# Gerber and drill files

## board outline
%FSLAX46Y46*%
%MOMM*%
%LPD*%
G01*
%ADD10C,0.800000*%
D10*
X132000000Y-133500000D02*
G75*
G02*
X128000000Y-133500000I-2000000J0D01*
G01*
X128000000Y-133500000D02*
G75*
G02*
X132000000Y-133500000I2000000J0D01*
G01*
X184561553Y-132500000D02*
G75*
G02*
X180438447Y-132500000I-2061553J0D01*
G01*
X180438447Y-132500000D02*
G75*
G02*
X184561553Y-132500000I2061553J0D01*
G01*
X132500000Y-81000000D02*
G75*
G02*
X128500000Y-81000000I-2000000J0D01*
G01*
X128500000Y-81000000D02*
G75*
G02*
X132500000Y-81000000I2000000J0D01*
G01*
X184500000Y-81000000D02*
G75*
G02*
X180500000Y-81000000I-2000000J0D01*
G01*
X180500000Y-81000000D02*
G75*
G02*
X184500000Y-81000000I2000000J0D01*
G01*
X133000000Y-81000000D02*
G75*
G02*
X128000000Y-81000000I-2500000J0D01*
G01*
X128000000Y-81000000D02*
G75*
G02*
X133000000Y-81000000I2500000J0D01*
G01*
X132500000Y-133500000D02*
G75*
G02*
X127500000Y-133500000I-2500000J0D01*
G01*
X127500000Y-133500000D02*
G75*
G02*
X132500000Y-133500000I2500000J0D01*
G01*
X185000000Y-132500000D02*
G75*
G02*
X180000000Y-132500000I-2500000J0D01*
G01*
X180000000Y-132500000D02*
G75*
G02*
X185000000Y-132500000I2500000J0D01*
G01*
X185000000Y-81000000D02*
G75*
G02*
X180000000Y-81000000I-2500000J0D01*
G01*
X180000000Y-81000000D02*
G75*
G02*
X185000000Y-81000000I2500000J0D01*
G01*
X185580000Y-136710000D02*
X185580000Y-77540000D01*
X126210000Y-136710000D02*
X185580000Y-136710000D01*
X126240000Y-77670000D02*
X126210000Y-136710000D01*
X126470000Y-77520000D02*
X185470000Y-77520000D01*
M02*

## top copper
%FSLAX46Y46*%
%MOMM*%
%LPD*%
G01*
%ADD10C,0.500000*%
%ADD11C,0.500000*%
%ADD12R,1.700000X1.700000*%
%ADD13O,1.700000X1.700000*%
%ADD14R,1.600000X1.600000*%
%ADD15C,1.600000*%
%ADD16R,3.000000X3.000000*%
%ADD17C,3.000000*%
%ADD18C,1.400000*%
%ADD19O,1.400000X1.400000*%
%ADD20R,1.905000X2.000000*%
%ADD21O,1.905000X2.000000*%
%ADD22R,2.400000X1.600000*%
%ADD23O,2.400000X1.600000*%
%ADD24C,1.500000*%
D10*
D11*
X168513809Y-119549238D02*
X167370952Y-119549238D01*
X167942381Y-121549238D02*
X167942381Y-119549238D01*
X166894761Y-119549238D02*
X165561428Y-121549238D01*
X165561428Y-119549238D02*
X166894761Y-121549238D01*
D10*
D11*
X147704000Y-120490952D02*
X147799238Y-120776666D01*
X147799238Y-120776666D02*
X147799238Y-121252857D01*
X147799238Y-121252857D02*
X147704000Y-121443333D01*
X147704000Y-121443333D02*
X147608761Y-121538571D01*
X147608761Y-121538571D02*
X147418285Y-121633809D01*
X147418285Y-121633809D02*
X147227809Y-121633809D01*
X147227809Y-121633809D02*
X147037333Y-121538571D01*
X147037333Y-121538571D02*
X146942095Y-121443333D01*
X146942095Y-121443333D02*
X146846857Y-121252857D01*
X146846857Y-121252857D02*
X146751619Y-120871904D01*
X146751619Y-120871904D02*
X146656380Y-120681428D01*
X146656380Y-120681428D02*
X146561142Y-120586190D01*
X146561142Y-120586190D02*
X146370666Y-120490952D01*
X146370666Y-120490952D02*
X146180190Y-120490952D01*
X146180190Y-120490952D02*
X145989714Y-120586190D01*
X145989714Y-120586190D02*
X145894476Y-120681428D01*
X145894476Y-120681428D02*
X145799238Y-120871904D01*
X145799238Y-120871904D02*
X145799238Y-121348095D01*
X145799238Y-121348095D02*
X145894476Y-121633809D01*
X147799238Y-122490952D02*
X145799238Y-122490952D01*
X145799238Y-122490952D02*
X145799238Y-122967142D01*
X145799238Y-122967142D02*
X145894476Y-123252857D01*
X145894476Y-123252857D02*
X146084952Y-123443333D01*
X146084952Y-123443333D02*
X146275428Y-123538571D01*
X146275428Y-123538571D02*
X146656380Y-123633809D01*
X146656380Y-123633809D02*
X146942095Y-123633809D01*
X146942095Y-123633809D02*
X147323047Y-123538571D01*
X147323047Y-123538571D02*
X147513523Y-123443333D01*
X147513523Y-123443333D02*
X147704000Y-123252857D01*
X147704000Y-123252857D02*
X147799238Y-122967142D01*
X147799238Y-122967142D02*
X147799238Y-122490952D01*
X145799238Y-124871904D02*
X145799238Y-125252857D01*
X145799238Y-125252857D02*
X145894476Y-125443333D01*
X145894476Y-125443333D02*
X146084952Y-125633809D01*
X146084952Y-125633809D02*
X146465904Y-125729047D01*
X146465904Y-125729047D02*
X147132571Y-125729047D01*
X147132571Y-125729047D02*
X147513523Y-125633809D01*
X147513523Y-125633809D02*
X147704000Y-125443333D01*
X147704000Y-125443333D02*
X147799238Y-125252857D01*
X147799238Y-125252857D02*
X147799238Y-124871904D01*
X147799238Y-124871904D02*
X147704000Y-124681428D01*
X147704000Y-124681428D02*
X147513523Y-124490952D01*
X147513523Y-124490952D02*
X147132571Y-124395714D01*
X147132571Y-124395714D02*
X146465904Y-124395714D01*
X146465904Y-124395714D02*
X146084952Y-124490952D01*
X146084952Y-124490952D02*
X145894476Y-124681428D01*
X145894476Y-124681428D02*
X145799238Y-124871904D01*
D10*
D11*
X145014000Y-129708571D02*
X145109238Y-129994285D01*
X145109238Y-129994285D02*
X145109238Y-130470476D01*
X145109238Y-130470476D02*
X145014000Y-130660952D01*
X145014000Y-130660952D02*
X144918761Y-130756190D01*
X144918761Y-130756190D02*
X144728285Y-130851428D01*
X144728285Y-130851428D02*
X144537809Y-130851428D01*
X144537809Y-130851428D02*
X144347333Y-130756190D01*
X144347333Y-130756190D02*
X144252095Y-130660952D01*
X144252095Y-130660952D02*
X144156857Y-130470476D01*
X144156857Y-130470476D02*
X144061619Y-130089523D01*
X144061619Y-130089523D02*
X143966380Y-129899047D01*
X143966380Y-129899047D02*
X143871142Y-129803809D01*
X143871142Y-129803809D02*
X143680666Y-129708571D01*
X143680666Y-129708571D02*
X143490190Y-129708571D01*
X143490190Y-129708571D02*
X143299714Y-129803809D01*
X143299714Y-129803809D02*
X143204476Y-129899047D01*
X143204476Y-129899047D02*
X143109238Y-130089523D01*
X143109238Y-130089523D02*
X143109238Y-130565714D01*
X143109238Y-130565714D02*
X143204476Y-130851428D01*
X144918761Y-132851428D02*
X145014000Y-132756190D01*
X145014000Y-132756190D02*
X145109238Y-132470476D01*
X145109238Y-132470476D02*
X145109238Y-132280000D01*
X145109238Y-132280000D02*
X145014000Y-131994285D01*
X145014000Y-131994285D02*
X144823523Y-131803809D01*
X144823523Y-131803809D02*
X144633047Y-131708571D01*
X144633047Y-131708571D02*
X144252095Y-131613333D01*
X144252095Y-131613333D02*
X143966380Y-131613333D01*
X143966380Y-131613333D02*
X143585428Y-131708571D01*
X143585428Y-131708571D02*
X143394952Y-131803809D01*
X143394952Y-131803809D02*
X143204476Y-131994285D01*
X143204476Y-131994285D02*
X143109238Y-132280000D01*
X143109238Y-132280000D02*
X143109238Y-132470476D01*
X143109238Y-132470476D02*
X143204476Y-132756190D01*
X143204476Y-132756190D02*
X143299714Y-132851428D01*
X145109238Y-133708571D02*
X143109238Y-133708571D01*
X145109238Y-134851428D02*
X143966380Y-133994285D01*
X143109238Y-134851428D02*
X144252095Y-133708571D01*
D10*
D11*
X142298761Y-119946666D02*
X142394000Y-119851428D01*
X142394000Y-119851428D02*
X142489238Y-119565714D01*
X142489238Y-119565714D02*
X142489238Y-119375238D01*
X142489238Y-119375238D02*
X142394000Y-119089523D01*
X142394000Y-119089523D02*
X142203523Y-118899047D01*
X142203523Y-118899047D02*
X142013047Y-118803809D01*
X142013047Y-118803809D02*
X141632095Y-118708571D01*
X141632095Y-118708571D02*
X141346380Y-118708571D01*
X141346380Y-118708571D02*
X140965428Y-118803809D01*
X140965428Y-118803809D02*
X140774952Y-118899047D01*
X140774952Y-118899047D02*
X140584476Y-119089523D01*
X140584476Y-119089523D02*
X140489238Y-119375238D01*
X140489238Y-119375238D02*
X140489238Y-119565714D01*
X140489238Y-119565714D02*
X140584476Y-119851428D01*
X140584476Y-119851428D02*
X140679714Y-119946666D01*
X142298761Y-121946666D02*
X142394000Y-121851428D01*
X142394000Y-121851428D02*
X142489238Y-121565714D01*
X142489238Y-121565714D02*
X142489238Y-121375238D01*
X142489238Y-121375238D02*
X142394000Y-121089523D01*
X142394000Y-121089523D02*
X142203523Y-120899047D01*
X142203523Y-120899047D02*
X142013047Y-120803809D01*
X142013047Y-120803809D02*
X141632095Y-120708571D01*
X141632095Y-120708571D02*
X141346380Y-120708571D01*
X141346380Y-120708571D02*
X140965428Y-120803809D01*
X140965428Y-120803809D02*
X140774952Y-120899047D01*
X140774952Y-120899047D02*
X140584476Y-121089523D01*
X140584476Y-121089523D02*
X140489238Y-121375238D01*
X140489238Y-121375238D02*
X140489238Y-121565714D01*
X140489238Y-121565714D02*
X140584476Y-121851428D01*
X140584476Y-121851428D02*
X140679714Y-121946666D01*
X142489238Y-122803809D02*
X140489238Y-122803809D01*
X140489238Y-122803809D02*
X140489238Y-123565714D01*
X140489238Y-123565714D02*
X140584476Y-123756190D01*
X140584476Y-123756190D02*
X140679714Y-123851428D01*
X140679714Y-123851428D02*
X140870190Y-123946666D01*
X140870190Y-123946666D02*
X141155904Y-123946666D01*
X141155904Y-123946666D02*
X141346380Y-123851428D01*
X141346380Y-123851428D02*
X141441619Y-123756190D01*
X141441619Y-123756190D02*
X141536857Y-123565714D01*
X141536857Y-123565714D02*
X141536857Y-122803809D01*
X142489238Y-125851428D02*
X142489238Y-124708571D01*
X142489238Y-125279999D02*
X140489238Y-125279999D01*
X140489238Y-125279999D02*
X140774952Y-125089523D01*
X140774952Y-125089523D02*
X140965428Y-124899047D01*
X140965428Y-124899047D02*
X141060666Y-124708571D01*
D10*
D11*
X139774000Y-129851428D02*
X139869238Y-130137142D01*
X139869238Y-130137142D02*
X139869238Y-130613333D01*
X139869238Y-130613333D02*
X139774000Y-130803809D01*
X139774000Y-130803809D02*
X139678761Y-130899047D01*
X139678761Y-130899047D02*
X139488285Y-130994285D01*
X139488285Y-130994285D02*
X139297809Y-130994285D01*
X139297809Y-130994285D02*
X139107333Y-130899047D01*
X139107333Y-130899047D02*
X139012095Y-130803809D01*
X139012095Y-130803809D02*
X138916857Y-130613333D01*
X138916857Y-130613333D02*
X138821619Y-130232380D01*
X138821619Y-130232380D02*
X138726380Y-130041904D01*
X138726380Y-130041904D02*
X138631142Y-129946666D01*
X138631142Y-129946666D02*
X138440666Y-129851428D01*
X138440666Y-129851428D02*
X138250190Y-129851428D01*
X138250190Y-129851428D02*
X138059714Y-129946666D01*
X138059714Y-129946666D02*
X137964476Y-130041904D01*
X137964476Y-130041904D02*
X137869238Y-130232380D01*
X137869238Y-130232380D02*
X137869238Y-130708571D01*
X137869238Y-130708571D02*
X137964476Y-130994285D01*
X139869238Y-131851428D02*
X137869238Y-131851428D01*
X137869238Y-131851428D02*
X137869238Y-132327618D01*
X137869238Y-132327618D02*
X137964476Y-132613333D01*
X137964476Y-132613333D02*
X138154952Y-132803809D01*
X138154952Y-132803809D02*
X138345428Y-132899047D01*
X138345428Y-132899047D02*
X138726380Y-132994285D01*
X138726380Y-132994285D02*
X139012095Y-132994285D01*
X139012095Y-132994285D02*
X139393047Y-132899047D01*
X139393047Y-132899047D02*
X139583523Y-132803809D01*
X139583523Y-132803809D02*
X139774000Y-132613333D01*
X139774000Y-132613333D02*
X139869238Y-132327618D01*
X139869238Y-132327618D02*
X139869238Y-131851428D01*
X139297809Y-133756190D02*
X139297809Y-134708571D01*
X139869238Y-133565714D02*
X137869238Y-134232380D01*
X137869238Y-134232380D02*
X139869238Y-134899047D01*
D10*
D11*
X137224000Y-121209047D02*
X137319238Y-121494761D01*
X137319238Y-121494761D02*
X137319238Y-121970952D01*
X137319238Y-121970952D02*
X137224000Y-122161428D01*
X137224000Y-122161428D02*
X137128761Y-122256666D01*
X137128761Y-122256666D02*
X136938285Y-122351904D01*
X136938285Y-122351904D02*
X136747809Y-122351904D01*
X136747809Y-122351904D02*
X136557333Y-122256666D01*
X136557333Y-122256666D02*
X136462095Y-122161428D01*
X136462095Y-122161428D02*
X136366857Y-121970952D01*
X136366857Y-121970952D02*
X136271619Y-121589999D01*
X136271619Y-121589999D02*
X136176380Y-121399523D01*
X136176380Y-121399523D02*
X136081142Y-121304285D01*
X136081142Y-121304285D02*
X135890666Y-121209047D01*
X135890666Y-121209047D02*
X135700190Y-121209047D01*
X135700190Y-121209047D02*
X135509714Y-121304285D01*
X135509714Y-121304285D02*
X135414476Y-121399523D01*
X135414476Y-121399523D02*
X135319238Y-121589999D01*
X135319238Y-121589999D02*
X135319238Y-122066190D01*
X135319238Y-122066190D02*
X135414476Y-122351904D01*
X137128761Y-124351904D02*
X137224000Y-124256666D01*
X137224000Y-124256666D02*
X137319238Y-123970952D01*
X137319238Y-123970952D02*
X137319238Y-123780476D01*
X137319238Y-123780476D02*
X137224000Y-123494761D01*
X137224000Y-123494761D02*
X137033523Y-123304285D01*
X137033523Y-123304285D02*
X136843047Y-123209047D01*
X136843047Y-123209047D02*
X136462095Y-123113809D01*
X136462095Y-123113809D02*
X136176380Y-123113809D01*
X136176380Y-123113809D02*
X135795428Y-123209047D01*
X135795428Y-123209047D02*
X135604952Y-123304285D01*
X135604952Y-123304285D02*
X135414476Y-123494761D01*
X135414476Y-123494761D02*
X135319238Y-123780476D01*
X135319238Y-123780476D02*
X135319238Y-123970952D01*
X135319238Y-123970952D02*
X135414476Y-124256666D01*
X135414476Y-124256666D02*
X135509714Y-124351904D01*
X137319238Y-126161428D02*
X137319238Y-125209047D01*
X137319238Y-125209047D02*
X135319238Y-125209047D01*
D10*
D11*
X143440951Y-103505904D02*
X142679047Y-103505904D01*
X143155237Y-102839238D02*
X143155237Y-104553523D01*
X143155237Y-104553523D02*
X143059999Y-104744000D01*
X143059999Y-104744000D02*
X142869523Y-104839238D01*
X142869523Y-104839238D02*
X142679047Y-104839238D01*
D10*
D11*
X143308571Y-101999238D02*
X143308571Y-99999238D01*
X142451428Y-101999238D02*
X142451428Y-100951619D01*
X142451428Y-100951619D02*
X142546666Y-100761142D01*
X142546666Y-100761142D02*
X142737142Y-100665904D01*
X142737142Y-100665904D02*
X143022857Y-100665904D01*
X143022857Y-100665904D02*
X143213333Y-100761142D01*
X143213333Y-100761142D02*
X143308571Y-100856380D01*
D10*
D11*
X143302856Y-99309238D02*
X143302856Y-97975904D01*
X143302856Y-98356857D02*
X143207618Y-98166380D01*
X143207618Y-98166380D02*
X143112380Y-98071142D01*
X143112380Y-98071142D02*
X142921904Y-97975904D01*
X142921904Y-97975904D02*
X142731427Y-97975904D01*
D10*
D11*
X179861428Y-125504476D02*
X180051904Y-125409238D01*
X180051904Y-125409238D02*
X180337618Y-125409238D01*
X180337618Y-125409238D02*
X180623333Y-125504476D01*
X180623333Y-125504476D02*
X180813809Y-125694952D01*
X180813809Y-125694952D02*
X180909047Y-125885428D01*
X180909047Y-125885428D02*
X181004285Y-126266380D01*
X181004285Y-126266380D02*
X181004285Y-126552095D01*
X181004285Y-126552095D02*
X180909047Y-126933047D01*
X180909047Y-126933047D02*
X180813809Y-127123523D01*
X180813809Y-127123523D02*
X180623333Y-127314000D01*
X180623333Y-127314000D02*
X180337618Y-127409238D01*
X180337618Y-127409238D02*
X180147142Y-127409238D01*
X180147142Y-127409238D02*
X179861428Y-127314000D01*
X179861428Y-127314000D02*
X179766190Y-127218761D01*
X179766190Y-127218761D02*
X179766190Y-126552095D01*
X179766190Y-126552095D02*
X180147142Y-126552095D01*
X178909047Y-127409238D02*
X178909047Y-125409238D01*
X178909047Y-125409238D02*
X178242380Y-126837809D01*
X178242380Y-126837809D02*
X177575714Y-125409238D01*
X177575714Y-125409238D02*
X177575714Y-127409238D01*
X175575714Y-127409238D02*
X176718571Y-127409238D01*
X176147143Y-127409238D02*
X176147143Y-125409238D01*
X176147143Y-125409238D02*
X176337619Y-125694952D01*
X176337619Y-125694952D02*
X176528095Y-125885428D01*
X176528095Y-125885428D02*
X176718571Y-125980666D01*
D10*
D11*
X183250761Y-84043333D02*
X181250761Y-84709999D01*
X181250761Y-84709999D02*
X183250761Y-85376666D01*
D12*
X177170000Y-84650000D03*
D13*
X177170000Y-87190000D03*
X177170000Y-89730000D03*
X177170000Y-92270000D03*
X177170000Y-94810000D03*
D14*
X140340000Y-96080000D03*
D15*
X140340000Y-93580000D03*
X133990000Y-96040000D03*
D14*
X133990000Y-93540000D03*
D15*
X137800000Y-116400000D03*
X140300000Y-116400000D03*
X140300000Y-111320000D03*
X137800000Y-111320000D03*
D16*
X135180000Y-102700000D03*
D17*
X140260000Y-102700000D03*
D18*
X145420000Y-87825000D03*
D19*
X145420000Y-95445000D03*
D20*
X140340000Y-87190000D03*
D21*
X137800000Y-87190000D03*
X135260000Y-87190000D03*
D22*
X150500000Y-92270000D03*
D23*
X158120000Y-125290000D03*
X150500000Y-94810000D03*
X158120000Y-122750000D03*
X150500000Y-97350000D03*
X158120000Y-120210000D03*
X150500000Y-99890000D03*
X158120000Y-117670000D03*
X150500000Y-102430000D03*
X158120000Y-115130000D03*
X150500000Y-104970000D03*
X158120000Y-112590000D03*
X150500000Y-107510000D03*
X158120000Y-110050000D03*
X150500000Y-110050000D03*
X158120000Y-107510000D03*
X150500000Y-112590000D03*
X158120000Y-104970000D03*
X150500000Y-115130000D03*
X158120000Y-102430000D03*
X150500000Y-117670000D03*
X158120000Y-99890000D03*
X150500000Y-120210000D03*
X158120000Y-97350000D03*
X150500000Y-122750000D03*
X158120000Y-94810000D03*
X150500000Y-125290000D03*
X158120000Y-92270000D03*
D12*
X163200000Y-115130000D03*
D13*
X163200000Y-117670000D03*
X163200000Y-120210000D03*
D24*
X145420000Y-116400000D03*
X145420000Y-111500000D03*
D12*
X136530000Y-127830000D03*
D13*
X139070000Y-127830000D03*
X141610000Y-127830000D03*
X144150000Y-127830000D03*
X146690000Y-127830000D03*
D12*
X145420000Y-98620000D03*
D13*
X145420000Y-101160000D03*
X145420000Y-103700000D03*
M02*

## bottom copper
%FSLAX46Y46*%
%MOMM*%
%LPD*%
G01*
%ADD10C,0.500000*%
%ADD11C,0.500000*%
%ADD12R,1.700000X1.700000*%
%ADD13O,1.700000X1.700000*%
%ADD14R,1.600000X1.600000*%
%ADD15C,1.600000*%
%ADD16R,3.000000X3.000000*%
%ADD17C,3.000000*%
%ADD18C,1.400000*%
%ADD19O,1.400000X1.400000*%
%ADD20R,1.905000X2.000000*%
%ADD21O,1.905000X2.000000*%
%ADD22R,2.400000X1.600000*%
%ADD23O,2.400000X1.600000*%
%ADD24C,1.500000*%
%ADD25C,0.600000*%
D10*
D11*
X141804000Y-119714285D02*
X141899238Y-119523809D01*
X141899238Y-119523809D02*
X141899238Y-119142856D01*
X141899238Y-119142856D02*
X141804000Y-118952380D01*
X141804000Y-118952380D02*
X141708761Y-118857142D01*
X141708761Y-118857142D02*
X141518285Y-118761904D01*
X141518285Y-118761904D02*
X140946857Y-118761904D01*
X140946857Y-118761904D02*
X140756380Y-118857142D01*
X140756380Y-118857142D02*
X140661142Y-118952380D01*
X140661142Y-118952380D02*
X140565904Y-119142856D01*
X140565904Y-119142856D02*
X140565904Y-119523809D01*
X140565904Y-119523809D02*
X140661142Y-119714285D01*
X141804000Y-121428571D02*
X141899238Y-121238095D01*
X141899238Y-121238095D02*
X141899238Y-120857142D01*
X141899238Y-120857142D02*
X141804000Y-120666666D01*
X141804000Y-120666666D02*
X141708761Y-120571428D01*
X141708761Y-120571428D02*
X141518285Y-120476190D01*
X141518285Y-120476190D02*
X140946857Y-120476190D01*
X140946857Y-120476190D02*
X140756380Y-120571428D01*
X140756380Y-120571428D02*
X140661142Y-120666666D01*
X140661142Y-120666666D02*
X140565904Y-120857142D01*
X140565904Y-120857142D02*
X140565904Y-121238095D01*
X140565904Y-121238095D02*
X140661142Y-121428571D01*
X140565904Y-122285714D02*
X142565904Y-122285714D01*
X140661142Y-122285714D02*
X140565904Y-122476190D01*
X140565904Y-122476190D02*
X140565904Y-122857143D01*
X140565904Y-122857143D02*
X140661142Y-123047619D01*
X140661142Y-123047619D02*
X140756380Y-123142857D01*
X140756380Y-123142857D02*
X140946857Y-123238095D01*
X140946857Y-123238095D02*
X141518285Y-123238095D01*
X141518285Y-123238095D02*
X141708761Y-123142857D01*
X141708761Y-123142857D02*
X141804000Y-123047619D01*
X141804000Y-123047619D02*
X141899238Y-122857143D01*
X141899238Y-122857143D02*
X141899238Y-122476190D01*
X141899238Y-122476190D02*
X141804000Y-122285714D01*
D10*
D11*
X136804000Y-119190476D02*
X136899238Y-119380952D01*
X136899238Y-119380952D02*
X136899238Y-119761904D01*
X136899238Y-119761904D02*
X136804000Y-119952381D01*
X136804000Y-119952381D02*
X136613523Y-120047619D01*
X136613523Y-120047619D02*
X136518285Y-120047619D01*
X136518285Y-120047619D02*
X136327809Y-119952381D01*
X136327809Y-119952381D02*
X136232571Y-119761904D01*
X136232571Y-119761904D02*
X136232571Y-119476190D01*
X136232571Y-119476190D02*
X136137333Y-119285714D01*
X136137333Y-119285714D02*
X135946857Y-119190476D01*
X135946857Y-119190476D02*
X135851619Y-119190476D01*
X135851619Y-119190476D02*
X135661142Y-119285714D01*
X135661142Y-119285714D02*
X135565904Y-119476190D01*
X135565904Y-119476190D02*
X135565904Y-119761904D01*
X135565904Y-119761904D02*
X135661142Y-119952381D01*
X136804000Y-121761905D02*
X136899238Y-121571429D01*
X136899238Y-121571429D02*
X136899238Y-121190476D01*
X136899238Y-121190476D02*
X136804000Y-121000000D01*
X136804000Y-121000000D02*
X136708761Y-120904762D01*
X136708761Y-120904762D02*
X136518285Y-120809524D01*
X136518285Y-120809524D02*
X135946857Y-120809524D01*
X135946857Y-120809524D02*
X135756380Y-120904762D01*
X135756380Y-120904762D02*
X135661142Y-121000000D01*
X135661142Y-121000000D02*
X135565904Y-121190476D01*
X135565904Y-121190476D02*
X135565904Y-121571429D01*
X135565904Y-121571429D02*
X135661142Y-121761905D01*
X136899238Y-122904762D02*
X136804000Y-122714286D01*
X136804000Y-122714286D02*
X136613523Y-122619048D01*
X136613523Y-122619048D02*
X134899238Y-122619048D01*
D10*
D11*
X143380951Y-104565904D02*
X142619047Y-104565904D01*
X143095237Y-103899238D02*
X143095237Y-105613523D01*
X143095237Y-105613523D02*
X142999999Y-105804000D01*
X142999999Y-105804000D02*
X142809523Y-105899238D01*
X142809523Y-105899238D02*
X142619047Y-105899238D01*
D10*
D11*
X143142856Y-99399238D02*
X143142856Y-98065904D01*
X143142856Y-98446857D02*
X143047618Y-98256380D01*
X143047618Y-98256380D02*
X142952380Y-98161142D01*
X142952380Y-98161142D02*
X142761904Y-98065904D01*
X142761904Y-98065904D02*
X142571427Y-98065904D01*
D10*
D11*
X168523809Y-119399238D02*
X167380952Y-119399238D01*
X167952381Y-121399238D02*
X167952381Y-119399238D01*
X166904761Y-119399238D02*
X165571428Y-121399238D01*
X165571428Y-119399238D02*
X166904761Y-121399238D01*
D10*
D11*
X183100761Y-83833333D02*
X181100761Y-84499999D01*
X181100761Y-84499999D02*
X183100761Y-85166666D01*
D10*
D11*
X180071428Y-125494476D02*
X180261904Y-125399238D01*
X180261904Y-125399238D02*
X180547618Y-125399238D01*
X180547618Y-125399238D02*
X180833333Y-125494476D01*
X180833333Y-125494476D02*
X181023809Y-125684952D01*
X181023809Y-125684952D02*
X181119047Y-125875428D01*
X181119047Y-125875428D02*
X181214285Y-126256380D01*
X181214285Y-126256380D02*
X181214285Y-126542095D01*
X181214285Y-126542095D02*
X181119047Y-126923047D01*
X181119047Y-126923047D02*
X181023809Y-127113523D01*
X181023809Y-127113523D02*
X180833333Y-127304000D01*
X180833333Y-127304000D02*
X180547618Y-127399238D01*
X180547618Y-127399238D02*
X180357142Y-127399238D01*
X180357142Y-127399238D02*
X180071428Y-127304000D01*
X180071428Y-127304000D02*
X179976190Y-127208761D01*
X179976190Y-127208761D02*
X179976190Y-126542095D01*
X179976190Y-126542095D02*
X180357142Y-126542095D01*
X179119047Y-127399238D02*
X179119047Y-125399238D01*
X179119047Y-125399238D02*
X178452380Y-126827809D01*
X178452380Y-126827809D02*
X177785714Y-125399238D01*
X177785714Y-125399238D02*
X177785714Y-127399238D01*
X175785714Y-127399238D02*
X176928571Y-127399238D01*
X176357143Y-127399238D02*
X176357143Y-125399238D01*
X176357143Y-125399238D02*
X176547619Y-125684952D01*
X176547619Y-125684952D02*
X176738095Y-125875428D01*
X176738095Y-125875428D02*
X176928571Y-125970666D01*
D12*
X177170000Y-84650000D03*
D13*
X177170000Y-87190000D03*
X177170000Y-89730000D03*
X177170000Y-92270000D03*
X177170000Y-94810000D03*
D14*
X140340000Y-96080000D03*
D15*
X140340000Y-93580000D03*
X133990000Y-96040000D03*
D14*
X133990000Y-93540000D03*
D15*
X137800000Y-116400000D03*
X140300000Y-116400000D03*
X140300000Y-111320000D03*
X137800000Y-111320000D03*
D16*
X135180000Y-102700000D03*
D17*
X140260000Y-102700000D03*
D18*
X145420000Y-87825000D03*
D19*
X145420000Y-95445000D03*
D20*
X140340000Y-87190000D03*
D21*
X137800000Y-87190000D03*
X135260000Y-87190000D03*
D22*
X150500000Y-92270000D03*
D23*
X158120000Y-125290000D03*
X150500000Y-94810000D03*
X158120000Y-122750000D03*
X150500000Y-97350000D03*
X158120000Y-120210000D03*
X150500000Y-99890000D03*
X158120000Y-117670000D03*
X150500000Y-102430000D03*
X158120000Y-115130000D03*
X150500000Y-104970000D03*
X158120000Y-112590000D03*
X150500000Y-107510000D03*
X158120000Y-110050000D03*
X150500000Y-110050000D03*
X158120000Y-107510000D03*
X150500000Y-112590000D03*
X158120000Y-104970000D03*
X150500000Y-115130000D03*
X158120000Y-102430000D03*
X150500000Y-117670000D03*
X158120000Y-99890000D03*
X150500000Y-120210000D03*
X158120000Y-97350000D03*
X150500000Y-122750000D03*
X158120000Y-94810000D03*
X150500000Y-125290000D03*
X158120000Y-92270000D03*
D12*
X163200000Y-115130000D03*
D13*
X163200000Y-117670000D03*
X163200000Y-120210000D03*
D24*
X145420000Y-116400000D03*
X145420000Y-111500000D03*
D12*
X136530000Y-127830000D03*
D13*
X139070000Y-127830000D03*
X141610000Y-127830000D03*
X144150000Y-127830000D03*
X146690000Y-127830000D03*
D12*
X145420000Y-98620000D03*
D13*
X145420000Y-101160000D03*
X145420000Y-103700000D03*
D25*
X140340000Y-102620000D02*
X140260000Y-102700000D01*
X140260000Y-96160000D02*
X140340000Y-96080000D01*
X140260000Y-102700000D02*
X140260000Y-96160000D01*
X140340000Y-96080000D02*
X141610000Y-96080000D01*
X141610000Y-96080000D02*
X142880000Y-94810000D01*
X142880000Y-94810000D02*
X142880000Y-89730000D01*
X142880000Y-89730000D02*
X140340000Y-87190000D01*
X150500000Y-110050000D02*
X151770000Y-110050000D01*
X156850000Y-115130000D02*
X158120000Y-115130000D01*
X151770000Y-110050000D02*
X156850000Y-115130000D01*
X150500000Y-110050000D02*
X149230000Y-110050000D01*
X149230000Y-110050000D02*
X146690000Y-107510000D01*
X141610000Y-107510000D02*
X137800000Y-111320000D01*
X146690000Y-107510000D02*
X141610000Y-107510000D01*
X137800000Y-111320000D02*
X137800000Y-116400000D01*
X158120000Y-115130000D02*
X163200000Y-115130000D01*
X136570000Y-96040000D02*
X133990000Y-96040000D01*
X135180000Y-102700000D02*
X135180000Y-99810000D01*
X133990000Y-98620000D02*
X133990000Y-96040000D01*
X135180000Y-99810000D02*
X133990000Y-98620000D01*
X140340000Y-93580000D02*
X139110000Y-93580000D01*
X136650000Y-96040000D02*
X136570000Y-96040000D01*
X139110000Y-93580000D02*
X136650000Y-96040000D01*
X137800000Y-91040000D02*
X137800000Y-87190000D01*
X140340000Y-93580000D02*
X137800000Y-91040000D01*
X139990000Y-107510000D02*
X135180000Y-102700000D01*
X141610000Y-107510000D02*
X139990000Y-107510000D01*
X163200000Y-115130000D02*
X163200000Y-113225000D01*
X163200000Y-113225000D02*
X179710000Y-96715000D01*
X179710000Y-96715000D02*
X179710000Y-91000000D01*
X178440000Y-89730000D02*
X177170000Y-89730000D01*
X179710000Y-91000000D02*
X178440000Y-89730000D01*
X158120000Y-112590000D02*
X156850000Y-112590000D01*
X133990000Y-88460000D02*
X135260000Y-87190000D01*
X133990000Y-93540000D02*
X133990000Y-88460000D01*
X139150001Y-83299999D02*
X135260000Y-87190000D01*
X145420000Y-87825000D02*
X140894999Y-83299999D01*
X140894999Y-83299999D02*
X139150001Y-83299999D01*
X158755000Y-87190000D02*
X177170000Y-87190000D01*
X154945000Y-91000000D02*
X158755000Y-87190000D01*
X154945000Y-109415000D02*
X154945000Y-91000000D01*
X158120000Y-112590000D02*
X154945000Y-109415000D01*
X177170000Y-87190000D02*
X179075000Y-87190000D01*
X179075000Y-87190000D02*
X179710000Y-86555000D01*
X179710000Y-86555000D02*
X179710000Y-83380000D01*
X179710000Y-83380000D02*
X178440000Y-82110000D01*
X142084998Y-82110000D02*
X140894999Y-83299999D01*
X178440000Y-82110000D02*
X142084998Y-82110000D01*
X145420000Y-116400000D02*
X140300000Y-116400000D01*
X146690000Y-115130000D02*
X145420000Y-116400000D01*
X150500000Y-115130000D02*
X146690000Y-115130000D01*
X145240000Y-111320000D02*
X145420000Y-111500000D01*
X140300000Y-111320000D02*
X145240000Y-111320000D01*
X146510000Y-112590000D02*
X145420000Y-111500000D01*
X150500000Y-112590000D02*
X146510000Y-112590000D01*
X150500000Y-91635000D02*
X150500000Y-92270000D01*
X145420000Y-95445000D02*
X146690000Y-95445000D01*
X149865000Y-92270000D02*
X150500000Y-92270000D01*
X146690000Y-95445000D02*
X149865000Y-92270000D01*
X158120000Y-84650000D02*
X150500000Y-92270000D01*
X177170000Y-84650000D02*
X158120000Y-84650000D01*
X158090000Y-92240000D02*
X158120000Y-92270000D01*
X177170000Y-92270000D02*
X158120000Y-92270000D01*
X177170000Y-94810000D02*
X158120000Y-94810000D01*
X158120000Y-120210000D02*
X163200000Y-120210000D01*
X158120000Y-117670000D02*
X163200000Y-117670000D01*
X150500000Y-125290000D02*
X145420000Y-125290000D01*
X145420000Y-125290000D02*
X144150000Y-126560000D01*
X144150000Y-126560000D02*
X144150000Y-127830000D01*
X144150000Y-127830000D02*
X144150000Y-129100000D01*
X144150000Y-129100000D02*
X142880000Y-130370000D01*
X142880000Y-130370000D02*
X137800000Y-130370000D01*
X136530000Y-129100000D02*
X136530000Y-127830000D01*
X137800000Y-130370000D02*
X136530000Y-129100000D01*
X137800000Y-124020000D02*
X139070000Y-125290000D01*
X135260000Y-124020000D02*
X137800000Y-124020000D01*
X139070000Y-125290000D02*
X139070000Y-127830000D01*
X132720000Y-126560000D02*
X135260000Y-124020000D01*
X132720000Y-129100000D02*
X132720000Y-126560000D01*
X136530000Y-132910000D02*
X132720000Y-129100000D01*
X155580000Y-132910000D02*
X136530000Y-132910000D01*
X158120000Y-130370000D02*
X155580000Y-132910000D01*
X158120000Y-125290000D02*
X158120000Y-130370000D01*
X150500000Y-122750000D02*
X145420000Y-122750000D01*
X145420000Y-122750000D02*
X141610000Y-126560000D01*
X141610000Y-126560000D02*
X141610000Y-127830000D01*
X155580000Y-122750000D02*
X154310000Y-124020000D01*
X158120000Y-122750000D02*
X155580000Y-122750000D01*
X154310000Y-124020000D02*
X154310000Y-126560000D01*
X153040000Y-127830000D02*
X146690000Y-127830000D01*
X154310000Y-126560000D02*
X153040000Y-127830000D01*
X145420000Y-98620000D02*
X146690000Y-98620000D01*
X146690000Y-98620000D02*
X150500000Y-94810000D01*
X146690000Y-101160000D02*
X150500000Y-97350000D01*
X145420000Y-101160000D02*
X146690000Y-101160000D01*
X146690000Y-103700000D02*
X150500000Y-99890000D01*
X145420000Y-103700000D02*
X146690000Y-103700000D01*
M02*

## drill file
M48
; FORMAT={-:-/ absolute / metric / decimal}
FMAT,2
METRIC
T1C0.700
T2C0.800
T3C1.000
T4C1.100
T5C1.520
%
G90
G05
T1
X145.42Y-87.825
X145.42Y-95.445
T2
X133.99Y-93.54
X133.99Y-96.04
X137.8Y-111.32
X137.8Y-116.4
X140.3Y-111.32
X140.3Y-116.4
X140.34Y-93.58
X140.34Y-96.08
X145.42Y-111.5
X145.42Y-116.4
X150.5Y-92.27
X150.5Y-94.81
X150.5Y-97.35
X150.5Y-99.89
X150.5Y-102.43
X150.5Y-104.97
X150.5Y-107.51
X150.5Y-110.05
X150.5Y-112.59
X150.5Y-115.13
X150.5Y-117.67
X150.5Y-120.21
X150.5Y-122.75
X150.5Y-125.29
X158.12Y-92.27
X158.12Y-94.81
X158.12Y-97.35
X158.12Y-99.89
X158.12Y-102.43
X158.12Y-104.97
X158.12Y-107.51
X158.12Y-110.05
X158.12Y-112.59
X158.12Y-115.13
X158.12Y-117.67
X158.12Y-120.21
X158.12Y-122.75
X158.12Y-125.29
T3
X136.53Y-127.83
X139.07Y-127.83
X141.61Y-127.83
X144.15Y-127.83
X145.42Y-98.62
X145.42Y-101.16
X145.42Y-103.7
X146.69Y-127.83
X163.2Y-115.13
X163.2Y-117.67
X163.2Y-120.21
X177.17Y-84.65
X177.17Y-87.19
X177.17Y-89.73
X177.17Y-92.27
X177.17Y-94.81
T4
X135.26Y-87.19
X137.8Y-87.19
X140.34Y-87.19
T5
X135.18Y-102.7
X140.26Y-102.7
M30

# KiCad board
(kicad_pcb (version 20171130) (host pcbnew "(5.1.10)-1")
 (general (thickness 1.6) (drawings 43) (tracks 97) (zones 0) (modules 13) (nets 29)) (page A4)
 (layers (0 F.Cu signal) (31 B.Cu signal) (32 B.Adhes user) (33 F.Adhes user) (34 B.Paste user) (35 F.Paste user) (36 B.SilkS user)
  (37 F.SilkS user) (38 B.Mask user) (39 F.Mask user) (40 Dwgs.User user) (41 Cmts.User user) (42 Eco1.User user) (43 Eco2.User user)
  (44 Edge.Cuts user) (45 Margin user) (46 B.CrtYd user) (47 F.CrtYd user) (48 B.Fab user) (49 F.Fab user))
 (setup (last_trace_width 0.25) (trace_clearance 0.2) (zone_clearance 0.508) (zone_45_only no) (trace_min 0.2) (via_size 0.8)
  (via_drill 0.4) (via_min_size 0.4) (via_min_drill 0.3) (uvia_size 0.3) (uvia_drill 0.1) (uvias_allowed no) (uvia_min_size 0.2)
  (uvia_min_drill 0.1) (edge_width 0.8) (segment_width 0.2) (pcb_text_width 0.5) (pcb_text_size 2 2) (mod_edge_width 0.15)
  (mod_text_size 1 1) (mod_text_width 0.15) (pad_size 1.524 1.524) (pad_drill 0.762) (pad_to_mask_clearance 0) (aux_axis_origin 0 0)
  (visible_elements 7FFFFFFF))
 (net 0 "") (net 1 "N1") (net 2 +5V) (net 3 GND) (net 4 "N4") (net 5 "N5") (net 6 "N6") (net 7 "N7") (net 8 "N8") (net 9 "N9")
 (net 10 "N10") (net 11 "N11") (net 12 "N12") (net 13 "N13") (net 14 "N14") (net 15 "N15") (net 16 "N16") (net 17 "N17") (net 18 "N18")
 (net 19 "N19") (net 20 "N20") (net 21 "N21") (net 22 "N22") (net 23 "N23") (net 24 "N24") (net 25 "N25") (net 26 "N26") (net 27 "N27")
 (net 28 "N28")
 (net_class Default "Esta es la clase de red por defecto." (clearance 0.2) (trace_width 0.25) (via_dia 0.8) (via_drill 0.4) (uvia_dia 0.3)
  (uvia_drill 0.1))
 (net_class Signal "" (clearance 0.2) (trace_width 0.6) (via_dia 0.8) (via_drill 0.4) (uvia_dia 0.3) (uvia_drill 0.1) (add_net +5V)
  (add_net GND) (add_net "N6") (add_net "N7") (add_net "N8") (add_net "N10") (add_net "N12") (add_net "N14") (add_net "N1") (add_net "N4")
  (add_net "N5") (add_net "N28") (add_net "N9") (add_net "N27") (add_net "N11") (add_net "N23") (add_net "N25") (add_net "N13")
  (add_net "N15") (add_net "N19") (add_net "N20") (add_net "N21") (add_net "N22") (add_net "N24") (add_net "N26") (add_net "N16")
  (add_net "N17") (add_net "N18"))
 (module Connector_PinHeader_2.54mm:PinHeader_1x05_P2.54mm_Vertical (layer F.Cu) (at 177.17 84.65)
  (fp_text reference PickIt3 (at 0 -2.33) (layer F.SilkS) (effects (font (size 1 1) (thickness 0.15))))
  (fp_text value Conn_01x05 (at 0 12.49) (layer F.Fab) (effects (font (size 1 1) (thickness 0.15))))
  (pad 1 thru_hole rect (at 0 0) (size 1.7 1.7) (drill 1) (layers *.Cu *.Mask) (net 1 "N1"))
  (pad 2 thru_hole oval (at 0 2.54) (size 1.7 1.7) (drill 1) (layers *.Cu *.Mask) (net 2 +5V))
  (pad 3 thru_hole oval (at 0 5.08) (size 1.7 1.7) (drill 1) (layers *.Cu *.Mask) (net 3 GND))
  (pad 4 thru_hole oval (at 0 7.62) (size 1.7 1.7) (drill 1) (layers *.Cu *.Mask) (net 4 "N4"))
  (pad 5 thru_hole oval (at 0 10.16) (size 1.7 1.7) (drill 1) (layers *.Cu *.Mask) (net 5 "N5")))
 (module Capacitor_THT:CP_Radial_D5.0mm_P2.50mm (layer F.Cu) (at 140.34 96.08 90)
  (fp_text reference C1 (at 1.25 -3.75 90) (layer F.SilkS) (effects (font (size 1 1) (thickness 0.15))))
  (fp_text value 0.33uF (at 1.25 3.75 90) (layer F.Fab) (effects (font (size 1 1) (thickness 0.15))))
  (pad 1 thru_hole rect (at 0 0 90) (size 1.6 1.6) (drill 0.8) (layers *.Cu *.Mask) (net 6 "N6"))
  (pad 2 thru_hole circle (at 2.5 0 90) (size 1.6 1.6) (drill 0.8) (layers *.Cu *.Mask) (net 3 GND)))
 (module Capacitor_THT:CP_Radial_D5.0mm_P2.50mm (layer F.Cu) (at 133.99 93.54 270)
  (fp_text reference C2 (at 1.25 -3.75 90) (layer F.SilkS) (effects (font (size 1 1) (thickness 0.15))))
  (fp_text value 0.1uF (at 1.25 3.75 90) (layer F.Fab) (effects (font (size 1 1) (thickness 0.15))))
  (pad 2 thru_hole circle (at 2.5 0 270) (size 1.6 1.6) (drill 0.8) (layers *.Cu *.Mask) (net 3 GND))
  (pad 1 thru_hole rect (at 0 0 270) (size 1.6 1.6) (drill 0.8) (layers *.Cu *.Mask) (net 2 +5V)))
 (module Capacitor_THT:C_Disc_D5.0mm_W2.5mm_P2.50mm (layer F.Cu) (at 137.8 116.4)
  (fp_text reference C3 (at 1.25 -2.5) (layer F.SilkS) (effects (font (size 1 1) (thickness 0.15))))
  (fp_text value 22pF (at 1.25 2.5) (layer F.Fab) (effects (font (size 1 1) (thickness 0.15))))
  (pad 1 thru_hole circle (at 0 0) (size 1.6 1.6) (drill 0.8) (layers *.Cu *.Mask) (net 3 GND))
  (pad 2 thru_hole circle (at 2.5 0) (size 1.6 1.6) (drill 0.8) (layers *.Cu *.Mask) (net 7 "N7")))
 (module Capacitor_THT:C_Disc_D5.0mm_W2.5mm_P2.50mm (layer F.Cu) (at 137.8 111.32)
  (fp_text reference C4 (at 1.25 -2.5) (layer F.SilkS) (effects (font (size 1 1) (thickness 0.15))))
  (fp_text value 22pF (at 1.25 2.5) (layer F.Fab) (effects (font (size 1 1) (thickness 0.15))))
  (pad 2 thru_hole circle (at 2.5 0) (size 1.6 1.6) (drill 0.8) (layers *.Cu *.Mask) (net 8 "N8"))
  (pad 1 thru_hole circle (at 0 0) (size 1.6 1.6) (drill 0.8) (layers *.Cu *.Mask) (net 3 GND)))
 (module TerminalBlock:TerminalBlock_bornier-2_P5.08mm (layer F.Cu) (at 135.18 102.7)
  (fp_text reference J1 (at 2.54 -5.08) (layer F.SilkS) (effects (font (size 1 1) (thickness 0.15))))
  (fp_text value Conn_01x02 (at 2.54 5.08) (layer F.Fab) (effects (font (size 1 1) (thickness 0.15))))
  (pad 1 thru_hole rect (at 0 0) (size 3 3) (drill 1.52) (layers *.Cu *.Mask) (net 3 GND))
  (pad 2 thru_hole circle (at 5.08 0) (size 3 3) (drill 1.52) (layers *.Cu *.Mask) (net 6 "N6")))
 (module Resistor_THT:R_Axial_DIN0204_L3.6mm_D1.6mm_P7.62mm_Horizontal (layer F.Cu) (at 145.42 87.825 270)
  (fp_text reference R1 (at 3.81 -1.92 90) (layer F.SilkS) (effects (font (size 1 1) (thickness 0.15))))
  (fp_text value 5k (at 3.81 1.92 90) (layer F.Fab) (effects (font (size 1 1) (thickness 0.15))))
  (pad 1 thru_hole circle (at 0 0 270) (size 1.4 1.4) (drill 0.7) (layers *.Cu *.Mask) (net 2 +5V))
  (pad 2 thru_hole oval (at 7.62 0 270) (size 1.4 1.4) (drill 0.7) (layers *.Cu *.Mask) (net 1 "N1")))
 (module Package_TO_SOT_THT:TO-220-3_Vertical (layer F.Cu) (at 140.34 87.19 180)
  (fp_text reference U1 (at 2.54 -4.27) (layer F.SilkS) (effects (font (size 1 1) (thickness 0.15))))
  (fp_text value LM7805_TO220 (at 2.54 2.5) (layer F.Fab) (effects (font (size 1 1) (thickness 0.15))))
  (pad 1 thru_hole rect (at 0 0 180) (size 1.905 2) (drill 1.1) (layers *.Cu *.Mask) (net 6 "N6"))
  (pad 2 thru_hole oval (at 2.54 0 180) (size 1.905 2) (drill 1.1) (layers *.Cu *.Mask) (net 3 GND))
  (pad 3 thru_hole oval (at 5.08 0 180) (size 1.905 2) (drill 1.1) (layers *.Cu *.Mask) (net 2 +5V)))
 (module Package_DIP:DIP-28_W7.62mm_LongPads (layer F.Cu) (at 150.5 92.27)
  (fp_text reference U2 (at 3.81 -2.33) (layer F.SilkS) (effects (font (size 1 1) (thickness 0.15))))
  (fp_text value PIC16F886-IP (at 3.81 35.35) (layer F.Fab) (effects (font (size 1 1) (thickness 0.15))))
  (pad 1 thru_hole rect (at 0 0) (size 2.4 1.6) (drill 0.8) (layers *.Cu *.Mask) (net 1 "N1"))
  (pad 15 thru_hole oval (at 7.62 33.02) (size 2.4 1.6) (drill 0.8) (layers *.Cu *.Mask) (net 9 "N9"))
  (pad 2 thru_hole oval (at 0 2.54) (size 2.4 1.6) (drill 0.8) (layers *.Cu *.Mask) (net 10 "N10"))
  (pad 16 thru_hole oval (at 7.62 30.48) (size 2.4 1.6) (drill 0.8) (layers *.Cu *.Mask) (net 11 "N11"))
  (pad 3 thru_hole oval (at 0 5.08) (size 2.4 1.6) (drill 0.8) (layers *.Cu *.Mask) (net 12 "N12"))
  (pad 17 thru_hole oval (at 7.62 27.94) (size 2.4 1.6) (drill 0.8) (layers *.Cu *.Mask) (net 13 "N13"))
  (pad 4 thru_hole oval (at 0 7.62) (size 2.4 1.6) (drill 0.8) (layers *.Cu *.Mask) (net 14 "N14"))
  (pad 18 thru_hole oval (at 7.62 25.4) (size 2.4 1.6) (drill 0.8) (layers *.Cu *.Mask) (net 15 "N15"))
  (pad 5 thru_hole oval (at 0 10.16) (size 2.4 1.6) (drill 0.8) (layers *.Cu *.Mask) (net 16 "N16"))
  (pad 19 thru_hole oval (at 7.62 22.86) (size 2.4 1.6) (drill 0.8) (layers *.Cu *.Mask) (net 3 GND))
  (pad 6 thru_hole oval (at 0 12.7) (size 2.4 1.6) (drill 0.8) (layers *.Cu *.Mask) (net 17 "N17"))
  (pad 20 thru_hole oval (at 7.62 20.32) (size 2.4 1.6) (drill 0.8) (layers *.Cu *.Mask) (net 2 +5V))
  (pad 7 thru_hole oval (at 0 15.24) (size 2.4 1.6) (drill 0.8) (layers *.Cu *.Mask) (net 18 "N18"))
  (pad 21 thru_hole oval (at 7.62 17.78) (size 2.4 1.6) (drill 0.8) (layers *.Cu *.Mask) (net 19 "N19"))
  (pad 8 thru_hole oval (at 0 17.78) (size 2.4 1.6) (drill 0.8) (layers *.Cu *.Mask) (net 3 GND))
  (pad 22 thru_hole oval (at 7.62 15.24) (size 2.4 1.6) (drill 0.8) (layers *.Cu *.Mask) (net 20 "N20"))
  (pad 9 thru_hole oval (at 0 20.32) (size 2.4 1.6) (drill 0.8) (layers *.Cu *.Mask) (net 8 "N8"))
  (pad 23 thru_hole oval (at 7.62 12.7) (size 2.4 1.6) (drill 0.8) (layers *.Cu *.Mask) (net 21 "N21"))
  (pad 10 thru_hole oval (at 0 22.86) (size 2.4 1.6) (drill 0.8) (layers *.Cu *.Mask) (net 7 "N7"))
  (pad 24 thru_hole oval (at 7.62 10.16) (size 2.4 1.6) (drill 0.8) (layers *.Cu *.Mask) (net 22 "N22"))
  (pad 11 thru_hole oval (at 0 25.4) (size 2.4 1.6) (drill 0.8) (layers *.Cu *.Mask) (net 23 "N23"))
  (pad 25 thru_hole oval (at 7.62 7.62) (size 2.4 1.6) (drill 0.8) (layers *.Cu *.Mask) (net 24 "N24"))
  (pad 12 thru_hole oval (at 0 27.94) (size 2.4 1.6) (drill 0.8) (layers *.Cu *.Mask) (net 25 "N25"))
  (pad 26 thru_hole oval (at 7.62 5.08) (size 2.4 1.6) (drill 0.8) (layers *.Cu *.Mask) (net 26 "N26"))
  (pad 13 thru_hole oval (at 0 30.48) (size 2.4 1.6) (drill 0.8) (layers *.Cu *.Mask) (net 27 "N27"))
  (pad 27 thru_hole oval (at 7.62 2.54) (size 2.4 1.6) (drill 0.8) (layers *.Cu *.Mask) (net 5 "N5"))
  (pad 14 thru_hole oval (at 0 33.02) (size 2.4 1.6) (drill 0.8) (layers *.Cu *.Mask) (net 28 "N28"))
  (pad 28 thru_hole oval (at 7.62 0) (size 2.4 1.6) (drill 0.8) (layers *.Cu *.Mask) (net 4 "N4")))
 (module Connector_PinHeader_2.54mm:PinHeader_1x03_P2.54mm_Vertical (layer F.Cu) (at 163.2 115.13)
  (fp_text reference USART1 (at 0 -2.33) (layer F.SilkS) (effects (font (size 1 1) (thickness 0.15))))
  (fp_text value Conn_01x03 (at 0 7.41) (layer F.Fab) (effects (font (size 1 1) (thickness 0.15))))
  (pad 1 thru_hole rect (at 0 0) (size 1.7 1.7) (drill 1) (layers *.Cu *.Mask) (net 3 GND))
  (pad 2 thru_hole oval (at 0 2.54) (size 1.7 1.7) (drill 1) (layers *.Cu *.Mask) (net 15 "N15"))
  (pad 3 thru_hole oval (at 0 5.08) (size 1.7 1.7) (drill 1) (layers *.Cu *.Mask) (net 13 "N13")))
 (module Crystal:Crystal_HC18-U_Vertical (layer F.Cu) (at 145.42 116.4 90)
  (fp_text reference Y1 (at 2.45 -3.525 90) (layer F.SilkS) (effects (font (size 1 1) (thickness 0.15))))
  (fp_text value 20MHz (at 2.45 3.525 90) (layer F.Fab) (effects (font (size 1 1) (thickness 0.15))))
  (pad 1 thru_hole circle (at 0 0 90) (size 1.5 1.5) (drill 0.8) (layers *.Cu *.Mask) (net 7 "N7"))
  (pad 2 thru_hole circle (at 4.9 0 90) (size 1.5 1.5) (drill 0.8) (layers *.Cu *.Mask) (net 8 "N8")))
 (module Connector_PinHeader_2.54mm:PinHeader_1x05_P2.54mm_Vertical (layer F.Cu) (at 136.53 127.83 90)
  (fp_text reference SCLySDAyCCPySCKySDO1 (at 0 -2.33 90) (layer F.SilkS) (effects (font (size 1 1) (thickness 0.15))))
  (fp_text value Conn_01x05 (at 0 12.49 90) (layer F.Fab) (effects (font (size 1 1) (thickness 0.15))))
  (pad 1 thru_hole rect (at 0 0 90) (size 1.7 1.7) (drill 1) (layers *.Cu *.Mask) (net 28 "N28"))
  (pad 2 thru_hole oval (at 0 2.54 90) (size 1.7 1.7) (drill 1) (layers *.Cu *.Mask) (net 9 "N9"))
  (pad 3 thru_hole oval (at 0 5.08 90) (size 1.7 1.7) (drill 1) (layers *.Cu *.Mask) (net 27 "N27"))
  (pad 4 thru_hole oval (at 0 7.62 90) (size 1.7 1.7) (drill 1) (layers *.Cu *.Mask) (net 28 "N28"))
  (pad 5 thru_hole oval (at 0 10.16 90) (size 1.7 1.7) (drill 1) (layers *.Cu *.Mask) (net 11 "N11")))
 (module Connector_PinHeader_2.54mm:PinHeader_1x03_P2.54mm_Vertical (layer F.Cu) (at 145.42 98.62)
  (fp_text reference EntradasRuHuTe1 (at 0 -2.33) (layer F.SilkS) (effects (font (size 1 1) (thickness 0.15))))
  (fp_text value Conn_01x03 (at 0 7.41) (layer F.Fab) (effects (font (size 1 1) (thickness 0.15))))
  (pad 1 thru_hole rect (at 0 0) (size 1.7 1.7) (drill 1) (layers *.Cu *.Mask) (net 10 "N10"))
  (pad 2 thru_hole oval (at 0 2.54) (size 1.7 1.7) (drill 1) (layers *.Cu *.Mask) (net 12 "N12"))
  (pad 3 thru_hole oval (at 0 5.08) (size 1.7 1.7) (drill 1) (layers *.Cu *.Mask) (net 14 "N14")))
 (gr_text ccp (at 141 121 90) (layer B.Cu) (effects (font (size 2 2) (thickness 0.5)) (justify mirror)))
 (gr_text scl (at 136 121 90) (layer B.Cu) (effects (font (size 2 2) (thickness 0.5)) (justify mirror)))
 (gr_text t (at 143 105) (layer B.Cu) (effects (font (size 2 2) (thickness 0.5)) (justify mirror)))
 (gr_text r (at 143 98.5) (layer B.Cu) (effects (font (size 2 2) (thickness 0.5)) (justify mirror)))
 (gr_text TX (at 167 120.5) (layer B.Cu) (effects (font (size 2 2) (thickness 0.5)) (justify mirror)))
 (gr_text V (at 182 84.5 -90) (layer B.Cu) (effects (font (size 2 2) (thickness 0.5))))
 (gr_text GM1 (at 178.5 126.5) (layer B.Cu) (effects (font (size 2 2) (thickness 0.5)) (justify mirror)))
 (gr_circle (center 130 133.5) (end 132 133.5) (layer Edge.Cuts) (width 0.8))
 (gr_circle (center 182.5 132.5) (end 184.5 133) (layer Edge.Cuts) (width 0.8))
 (gr_circle (center 130.5 81) (end 132.5 81) (layer Edge.Cuts) (width 0.8))
 (gr_circle (center 182.5 81) (end 184.5 81) (layer Edge.Cuts) (width 0.8))
 (gr_circle (center 130.5 81) (end 133 81) (layer Edge.Cuts) (width 0.8))
 (gr_circle (center 130 133.5) (end 132.5 133.5) (layer Edge.Cuts) (width 0.8))
 (gr_circle (center 182.5 132.5) (end 185 132.5) (layer Edge.Cuts) (width 0.8))
 (gr_circle (center 182.5 81) (end 185 81) (layer Edge.Cuts) (width 0.8))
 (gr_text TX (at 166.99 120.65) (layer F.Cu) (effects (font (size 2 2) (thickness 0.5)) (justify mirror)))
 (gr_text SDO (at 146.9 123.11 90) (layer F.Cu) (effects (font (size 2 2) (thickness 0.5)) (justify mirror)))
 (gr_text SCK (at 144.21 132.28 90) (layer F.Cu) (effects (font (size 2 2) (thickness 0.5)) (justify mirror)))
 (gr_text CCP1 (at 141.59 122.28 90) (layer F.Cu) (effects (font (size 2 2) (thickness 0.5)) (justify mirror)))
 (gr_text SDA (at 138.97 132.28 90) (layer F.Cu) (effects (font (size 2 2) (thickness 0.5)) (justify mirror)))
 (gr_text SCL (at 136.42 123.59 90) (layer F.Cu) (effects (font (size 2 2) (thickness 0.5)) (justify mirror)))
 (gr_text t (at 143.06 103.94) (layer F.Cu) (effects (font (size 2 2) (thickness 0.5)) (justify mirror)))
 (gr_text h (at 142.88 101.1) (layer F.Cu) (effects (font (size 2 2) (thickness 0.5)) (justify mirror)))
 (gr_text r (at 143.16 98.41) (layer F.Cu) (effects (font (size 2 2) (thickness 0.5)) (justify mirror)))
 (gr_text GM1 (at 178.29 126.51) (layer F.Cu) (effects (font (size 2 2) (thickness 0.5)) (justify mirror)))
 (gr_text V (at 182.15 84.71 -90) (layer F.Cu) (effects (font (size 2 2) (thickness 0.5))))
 (gr_line (start 185.58 136.71) (end 185.58 77.54) (layer Edge.Cuts) (width 0.8))
 (gr_line (start 126.21 136.71) (end 185.58 136.71) (layer Edge.Cuts) (width 0.8))
 (gr_line (start 126.24 77.67) (end 126.21 136.71) (layer Edge.Cuts) (width 0.8))
 (gr_line (start 126.47 77.52) (end 185.47 77.52) (layer Edge.Cuts) (width 0.8))
 (segment (start 140.34 102.62) (end 140.26 102.7) (width 0.6) (layer B.Cu) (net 6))
 (segment (start 140.26 96.16) (end 140.34 96.08) (width 0.6) (layer B.Cu) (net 6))
 (segment (start 140.26 102.7) (end 140.26 96.16) (width 0.6) (layer B.Cu) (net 6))
 (segment (start 140.34 96.08) (end 141.61 96.08) (width 0.6) (layer B.Cu) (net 6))
 (segment (start 141.61 96.08) (end 142.88 94.81) (width 0.6) (layer B.Cu) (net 6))
 (segment (start 142.88 94.81) (end 142.88 89.73) (width 0.6) (layer B.Cu) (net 6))
 (segment (start 142.88 89.73) (end 140.34 87.19) (width 0.6) (layer B.Cu) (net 6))
 (segment (start 150.5 110.05) (end 151.77 110.05) (width 0.6) (layer B.Cu) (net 3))
 (segment (start 156.85 115.13) (end 158.12 115.13) (width 0.6) (layer B.Cu) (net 3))
 (segment (start 151.77 110.05) (end 156.85 115.13) (width 0.6) (layer B.Cu) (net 3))
 (segment (start 150.5 110.05) (end 149.23 110.05) (width 0.6) (layer B.Cu) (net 3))
 (segment (start 149.23 110.05) (end 146.69 107.51) (width 0.6) (layer B.Cu) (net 3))
 (segment (start 141.61 107.51) (end 137.8 111.32) (width 0.6) (layer B.Cu) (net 3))
 (segment (start 146.69 107.51) (end 141.61 107.51) (width 0.6) (layer B.Cu) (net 3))
 (segment (start 137.8 111.32) (end 137.8 116.4) (width 0.6) (layer B.Cu) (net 3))
 (segment (start 158.12 115.13) (end 163.2 115.13) (width 0.6) (layer B.Cu) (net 3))
 (segment (start 136.57 96.04) (end 133.99 96.04) (width 0.6) (layer B.Cu) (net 3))
 (segment (start 135.18 102.7) (end 135.18 99.81) (width 0.6) (layer B.Cu) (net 3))
 (segment (start 133.99 98.62) (end 133.99 96.04) (width 0.6) (layer B.Cu) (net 3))
 (segment (start 135.18 99.81) (end 133.99 98.62) (width 0.6) (layer B.Cu) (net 3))
 (segment (start 140.34 93.58) (end 139.11 93.58) (width 0.6) (layer B.Cu) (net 3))
 (segment (start 136.65 96.04) (end 136.57 96.04) (width 0.6) (layer B.Cu) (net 3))
 (segment (start 139.11 93.58) (end 136.65 96.04) (width 0.6) (layer B.Cu) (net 3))
 (segment (start 137.8 91.04) (end 137.8 87.19) (width 0.6) (layer B.Cu) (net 3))
 (segment (start 140.34 93.58) (end 137.8 91.04) (width 0.6) (layer B.Cu) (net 3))
 (segment (start 139.99 107.51) (end 135.18 102.7) (width 0.6) (layer B.Cu) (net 3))
 (segment (start 141.61 107.51) (end 139.99 107.51) (width 0.6) (layer B.Cu) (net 3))
 (segment (start 163.2 115.13) (end 163.2 113.225) (width 0.6) (layer B.Cu) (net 3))
 (segment (start 163.2 113.225) (end 179.71 96.715) (width 0.6) (layer B.Cu) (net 3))
 (segment (start 179.71 96.715) (end 179.71 91) (width 0.6) (layer B.Cu) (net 3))
 (segment (start 178.44 89.73) (end 177.17 89.73) (width 0.6) (layer B.Cu) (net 3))
 (segment (start 179.71 91) (end 178.44 89.73) (width 0.6) (layer B.Cu) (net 3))
 (segment (start 158.12 112.59) (end 156.85 112.59) (width 0.6) (layer B.Cu) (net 2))
 (segment (start 133.99 88.46) (end 135.26 87.19) (width 0.6) (layer B.Cu) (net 2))
 (segment (start 133.99 93.54) (end 133.99 88.46) (width 0.6) (layer B.Cu) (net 2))
 (segment (start 139.150001 83.299999) (end 135.26 87.19) (width 0.6) (layer B.Cu) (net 2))
 (segment (start 145.42 87.825) (end 140.894999 83.299999) (width 0.6) (layer B.Cu) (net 2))
 (segment (start 140.894999 83.299999) (end 139.150001 83.299999) (width 0.6) (layer B.Cu) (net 2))
 (segment (start 158.755 87.19) (end 177.17 87.19) (width 0.6) (layer B.Cu) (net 2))
 (segment (start 154.945 91) (end 158.755 87.19) (width 0.6) (layer B.Cu) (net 2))
 (segment (start 154.945 109.415) (end 154.945 91) (width 0.6) (layer B.Cu) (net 2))
 (segment (start 158.12 112.59) (end 154.945 109.415) (width 0.6) (layer B.Cu) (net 2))
 (segment (start 177.17 87.19) (end 179.075 87.19) (width 0.6) (layer B.Cu) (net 2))
 (segment (start 179.075 87.19) (end 179.71 86.555) (width 0.6) (layer B.Cu) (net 2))
 (segment (start 179.71 86.555) (end 179.71 83.38) (width 0.6) (layer B.Cu) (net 2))
 (segment (start 179.71 83.38) (end 178.44 82.11) (width 0.6) (layer B.Cu) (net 2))
 (segment (start 142.084998 82.11) (end 140.894999 83.299999) (width 0.6) (layer B.Cu) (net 2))
 (segment (start 178.44 82.11) (end 142.084998 82.11) (width 0.6) (layer B.Cu) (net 2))
 (segment (start 145.42 116.4) (end 140.3 116.4) (width 0.6) (layer B.Cu) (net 7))
 (segment (start 146.69 115.13) (end 145.42 116.4) (width 0.6) (layer B.Cu) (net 7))
 (segment (start 150.5 115.13) (end 146.69 115.13) (width 0.6) (layer B.Cu) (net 7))
 (segment (start 145.24 111.32) (end 145.42 111.5) (width 0.6) (layer B.Cu) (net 8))
 (segment (start 140.3 111.32) (end 145.24 111.32) (width 0.6) (layer B.Cu) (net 8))
 (segment (start 146.51 112.59) (end 145.42 111.5) (width 0.6) (layer B.Cu) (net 8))
 (segment (start 150.5 112.59) (end 146.51 112.59) (width 0.6) (layer B.Cu) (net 8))
 (segment (start 150.5 91.635) (end 150.5 92.27) (width 0.6) (layer B.Cu) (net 1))
 (segment (start 145.42 95.445) (end 146.69 95.445) (width 0.6) (layer B.Cu) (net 1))
 (segment (start 149.865 92.27) (end 150.5 92.27) (width 0.6) (layer B.Cu) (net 1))
 (segment (start 146.69 95.445) (end 149.865 92.27) (width 0.6) (layer B.Cu) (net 1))
 (segment (start 158.12 84.65) (end 150.5 92.27) (width 0.6) (layer B.Cu) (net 1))
 (segment (start 177.17 84.65) (end 158.12 84.65) (width 0.6) (layer B.Cu) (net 1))
 (segment (start 158.09 92.24) (end 158.12 92.27) (width 0.6) (layer B.Cu) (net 4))
 (segment (start 177.17 92.27) (end 158.12 92.27) (width 0.6) (layer B.Cu) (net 4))
 (segment (start 177.17 94.81) (end 158.12 94.81) (width 0.6) (layer B.Cu) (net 5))
 (segment (start 158.12 120.21) (end 163.2 120.21) (width 0.6) (layer B.Cu) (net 13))
 (segment (start 158.12 117.67) (end 163.2 117.67) (width 0.6) (layer B.Cu) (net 15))
 (segment (start 150.5 125.29) (end 145.42 125.29) (width 0.6) (layer B.Cu) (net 28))
 (segment (start 145.42 125.29) (end 144.15 126.56) (width 0.6) (layer B.Cu) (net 28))
 (segment (start 144.15 126.56) (end 144.15 127.83) (width 0.6) (layer B.Cu) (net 28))
 (segment (start 144.15 127.83) (end 144.15 129.1) (width 0.6) (layer B.Cu) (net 28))
 (segment (start 144.15 129.1) (end 142.88 130.37) (width 0.6) (layer B.Cu) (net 28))
 (segment (start 142.88 130.37) (end 137.8 130.37) (width 0.6) (layer B.Cu) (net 28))
 (segment (start 136.53 129.1) (end 136.53 127.83) (width 0.6) (layer B.Cu) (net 28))
 (segment (start 137.8 130.37) (end 136.53 129.1) (width 0.6) (layer B.Cu) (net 28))
 (segment (start 137.8 124.02) (end 139.07 125.29) (width 0.6) (layer B.Cu) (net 9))
 (segment (start 135.26 124.02) (end 137.8 124.02) (width 0.6) (layer B.Cu) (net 9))
 (segment (start 139.07 125.29) (end 139.07 127.83) (width 0.6) (layer B.Cu) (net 9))
 (segment (start 132.72 126.56) (end 135.26 124.02) (width 0.6) (layer B.Cu) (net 9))
 (segment (start 132.72 129.1) (end 132.72 126.56) (width 0.6) (layer B.Cu) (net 9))
 (segment (start 136.53 132.91) (end 132.72 129.1) (width 0.6) (layer B.Cu) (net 9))
 (segment (start 155.58 132.91) (end 136.53 132.91) (width 0.6) (layer B.Cu) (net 9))
 (segment (start 158.12 130.37) (end 155.58 132.91) (width 0.6) (layer B.Cu) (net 9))
 (segment (start 158.12 125.29) (end 158.12 130.37) (width 0.6) (layer B.Cu) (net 9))
 (segment (start 150.5 122.75) (end 145.42 122.75) (width 0.6) (layer B.Cu) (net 27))
 (segment (start 145.42 122.75) (end 141.61 126.56) (width 0.6) (layer B.Cu) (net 27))
 (segment (start 141.61 126.56) (end 141.61 127.83) (width 0.6) (layer B.Cu) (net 27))
 (segment (start 155.58 122.75) (end 154.31 124.02) (width 0.6) (layer B.Cu) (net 11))
 (segment (start 158.12 122.75) (end 155.58 122.75) (width 0.6) (layer B.Cu) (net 11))
 (segment (start 154.31 124.02) (end 154.31 126.56) (width 0.6) (layer B.Cu) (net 11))
 (segment (start 153.04 127.83) (end 146.69 127.83) (width 0.6) (layer B.Cu) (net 11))
 (segment (start 154.31 126.56) (end 153.04 127.83) (width 0.6) (layer B.Cu) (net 11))
 (segment (start 145.42 98.62) (end 146.69 98.62) (width 0.6) (layer B.Cu) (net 10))
 (segment (start 146.69 98.62) (end 150.5 94.81) (width 0.6) (layer B.Cu) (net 10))
 (segment (start 146.69 101.16) (end 150.5 97.35) (width 0.6) (layer B.Cu) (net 12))
 (segment (start 145.42 101.16) (end 146.69 101.16) (width 0.6) (layer B.Cu) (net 12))
 (segment (start 146.69 103.7) (end 150.5 99.89) (width 0.6) (layer B.Cu) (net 14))
 (segment (start 145.42 103.7) (end 146.69 103.7) (width 0.6) (layer B.Cu) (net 14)))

